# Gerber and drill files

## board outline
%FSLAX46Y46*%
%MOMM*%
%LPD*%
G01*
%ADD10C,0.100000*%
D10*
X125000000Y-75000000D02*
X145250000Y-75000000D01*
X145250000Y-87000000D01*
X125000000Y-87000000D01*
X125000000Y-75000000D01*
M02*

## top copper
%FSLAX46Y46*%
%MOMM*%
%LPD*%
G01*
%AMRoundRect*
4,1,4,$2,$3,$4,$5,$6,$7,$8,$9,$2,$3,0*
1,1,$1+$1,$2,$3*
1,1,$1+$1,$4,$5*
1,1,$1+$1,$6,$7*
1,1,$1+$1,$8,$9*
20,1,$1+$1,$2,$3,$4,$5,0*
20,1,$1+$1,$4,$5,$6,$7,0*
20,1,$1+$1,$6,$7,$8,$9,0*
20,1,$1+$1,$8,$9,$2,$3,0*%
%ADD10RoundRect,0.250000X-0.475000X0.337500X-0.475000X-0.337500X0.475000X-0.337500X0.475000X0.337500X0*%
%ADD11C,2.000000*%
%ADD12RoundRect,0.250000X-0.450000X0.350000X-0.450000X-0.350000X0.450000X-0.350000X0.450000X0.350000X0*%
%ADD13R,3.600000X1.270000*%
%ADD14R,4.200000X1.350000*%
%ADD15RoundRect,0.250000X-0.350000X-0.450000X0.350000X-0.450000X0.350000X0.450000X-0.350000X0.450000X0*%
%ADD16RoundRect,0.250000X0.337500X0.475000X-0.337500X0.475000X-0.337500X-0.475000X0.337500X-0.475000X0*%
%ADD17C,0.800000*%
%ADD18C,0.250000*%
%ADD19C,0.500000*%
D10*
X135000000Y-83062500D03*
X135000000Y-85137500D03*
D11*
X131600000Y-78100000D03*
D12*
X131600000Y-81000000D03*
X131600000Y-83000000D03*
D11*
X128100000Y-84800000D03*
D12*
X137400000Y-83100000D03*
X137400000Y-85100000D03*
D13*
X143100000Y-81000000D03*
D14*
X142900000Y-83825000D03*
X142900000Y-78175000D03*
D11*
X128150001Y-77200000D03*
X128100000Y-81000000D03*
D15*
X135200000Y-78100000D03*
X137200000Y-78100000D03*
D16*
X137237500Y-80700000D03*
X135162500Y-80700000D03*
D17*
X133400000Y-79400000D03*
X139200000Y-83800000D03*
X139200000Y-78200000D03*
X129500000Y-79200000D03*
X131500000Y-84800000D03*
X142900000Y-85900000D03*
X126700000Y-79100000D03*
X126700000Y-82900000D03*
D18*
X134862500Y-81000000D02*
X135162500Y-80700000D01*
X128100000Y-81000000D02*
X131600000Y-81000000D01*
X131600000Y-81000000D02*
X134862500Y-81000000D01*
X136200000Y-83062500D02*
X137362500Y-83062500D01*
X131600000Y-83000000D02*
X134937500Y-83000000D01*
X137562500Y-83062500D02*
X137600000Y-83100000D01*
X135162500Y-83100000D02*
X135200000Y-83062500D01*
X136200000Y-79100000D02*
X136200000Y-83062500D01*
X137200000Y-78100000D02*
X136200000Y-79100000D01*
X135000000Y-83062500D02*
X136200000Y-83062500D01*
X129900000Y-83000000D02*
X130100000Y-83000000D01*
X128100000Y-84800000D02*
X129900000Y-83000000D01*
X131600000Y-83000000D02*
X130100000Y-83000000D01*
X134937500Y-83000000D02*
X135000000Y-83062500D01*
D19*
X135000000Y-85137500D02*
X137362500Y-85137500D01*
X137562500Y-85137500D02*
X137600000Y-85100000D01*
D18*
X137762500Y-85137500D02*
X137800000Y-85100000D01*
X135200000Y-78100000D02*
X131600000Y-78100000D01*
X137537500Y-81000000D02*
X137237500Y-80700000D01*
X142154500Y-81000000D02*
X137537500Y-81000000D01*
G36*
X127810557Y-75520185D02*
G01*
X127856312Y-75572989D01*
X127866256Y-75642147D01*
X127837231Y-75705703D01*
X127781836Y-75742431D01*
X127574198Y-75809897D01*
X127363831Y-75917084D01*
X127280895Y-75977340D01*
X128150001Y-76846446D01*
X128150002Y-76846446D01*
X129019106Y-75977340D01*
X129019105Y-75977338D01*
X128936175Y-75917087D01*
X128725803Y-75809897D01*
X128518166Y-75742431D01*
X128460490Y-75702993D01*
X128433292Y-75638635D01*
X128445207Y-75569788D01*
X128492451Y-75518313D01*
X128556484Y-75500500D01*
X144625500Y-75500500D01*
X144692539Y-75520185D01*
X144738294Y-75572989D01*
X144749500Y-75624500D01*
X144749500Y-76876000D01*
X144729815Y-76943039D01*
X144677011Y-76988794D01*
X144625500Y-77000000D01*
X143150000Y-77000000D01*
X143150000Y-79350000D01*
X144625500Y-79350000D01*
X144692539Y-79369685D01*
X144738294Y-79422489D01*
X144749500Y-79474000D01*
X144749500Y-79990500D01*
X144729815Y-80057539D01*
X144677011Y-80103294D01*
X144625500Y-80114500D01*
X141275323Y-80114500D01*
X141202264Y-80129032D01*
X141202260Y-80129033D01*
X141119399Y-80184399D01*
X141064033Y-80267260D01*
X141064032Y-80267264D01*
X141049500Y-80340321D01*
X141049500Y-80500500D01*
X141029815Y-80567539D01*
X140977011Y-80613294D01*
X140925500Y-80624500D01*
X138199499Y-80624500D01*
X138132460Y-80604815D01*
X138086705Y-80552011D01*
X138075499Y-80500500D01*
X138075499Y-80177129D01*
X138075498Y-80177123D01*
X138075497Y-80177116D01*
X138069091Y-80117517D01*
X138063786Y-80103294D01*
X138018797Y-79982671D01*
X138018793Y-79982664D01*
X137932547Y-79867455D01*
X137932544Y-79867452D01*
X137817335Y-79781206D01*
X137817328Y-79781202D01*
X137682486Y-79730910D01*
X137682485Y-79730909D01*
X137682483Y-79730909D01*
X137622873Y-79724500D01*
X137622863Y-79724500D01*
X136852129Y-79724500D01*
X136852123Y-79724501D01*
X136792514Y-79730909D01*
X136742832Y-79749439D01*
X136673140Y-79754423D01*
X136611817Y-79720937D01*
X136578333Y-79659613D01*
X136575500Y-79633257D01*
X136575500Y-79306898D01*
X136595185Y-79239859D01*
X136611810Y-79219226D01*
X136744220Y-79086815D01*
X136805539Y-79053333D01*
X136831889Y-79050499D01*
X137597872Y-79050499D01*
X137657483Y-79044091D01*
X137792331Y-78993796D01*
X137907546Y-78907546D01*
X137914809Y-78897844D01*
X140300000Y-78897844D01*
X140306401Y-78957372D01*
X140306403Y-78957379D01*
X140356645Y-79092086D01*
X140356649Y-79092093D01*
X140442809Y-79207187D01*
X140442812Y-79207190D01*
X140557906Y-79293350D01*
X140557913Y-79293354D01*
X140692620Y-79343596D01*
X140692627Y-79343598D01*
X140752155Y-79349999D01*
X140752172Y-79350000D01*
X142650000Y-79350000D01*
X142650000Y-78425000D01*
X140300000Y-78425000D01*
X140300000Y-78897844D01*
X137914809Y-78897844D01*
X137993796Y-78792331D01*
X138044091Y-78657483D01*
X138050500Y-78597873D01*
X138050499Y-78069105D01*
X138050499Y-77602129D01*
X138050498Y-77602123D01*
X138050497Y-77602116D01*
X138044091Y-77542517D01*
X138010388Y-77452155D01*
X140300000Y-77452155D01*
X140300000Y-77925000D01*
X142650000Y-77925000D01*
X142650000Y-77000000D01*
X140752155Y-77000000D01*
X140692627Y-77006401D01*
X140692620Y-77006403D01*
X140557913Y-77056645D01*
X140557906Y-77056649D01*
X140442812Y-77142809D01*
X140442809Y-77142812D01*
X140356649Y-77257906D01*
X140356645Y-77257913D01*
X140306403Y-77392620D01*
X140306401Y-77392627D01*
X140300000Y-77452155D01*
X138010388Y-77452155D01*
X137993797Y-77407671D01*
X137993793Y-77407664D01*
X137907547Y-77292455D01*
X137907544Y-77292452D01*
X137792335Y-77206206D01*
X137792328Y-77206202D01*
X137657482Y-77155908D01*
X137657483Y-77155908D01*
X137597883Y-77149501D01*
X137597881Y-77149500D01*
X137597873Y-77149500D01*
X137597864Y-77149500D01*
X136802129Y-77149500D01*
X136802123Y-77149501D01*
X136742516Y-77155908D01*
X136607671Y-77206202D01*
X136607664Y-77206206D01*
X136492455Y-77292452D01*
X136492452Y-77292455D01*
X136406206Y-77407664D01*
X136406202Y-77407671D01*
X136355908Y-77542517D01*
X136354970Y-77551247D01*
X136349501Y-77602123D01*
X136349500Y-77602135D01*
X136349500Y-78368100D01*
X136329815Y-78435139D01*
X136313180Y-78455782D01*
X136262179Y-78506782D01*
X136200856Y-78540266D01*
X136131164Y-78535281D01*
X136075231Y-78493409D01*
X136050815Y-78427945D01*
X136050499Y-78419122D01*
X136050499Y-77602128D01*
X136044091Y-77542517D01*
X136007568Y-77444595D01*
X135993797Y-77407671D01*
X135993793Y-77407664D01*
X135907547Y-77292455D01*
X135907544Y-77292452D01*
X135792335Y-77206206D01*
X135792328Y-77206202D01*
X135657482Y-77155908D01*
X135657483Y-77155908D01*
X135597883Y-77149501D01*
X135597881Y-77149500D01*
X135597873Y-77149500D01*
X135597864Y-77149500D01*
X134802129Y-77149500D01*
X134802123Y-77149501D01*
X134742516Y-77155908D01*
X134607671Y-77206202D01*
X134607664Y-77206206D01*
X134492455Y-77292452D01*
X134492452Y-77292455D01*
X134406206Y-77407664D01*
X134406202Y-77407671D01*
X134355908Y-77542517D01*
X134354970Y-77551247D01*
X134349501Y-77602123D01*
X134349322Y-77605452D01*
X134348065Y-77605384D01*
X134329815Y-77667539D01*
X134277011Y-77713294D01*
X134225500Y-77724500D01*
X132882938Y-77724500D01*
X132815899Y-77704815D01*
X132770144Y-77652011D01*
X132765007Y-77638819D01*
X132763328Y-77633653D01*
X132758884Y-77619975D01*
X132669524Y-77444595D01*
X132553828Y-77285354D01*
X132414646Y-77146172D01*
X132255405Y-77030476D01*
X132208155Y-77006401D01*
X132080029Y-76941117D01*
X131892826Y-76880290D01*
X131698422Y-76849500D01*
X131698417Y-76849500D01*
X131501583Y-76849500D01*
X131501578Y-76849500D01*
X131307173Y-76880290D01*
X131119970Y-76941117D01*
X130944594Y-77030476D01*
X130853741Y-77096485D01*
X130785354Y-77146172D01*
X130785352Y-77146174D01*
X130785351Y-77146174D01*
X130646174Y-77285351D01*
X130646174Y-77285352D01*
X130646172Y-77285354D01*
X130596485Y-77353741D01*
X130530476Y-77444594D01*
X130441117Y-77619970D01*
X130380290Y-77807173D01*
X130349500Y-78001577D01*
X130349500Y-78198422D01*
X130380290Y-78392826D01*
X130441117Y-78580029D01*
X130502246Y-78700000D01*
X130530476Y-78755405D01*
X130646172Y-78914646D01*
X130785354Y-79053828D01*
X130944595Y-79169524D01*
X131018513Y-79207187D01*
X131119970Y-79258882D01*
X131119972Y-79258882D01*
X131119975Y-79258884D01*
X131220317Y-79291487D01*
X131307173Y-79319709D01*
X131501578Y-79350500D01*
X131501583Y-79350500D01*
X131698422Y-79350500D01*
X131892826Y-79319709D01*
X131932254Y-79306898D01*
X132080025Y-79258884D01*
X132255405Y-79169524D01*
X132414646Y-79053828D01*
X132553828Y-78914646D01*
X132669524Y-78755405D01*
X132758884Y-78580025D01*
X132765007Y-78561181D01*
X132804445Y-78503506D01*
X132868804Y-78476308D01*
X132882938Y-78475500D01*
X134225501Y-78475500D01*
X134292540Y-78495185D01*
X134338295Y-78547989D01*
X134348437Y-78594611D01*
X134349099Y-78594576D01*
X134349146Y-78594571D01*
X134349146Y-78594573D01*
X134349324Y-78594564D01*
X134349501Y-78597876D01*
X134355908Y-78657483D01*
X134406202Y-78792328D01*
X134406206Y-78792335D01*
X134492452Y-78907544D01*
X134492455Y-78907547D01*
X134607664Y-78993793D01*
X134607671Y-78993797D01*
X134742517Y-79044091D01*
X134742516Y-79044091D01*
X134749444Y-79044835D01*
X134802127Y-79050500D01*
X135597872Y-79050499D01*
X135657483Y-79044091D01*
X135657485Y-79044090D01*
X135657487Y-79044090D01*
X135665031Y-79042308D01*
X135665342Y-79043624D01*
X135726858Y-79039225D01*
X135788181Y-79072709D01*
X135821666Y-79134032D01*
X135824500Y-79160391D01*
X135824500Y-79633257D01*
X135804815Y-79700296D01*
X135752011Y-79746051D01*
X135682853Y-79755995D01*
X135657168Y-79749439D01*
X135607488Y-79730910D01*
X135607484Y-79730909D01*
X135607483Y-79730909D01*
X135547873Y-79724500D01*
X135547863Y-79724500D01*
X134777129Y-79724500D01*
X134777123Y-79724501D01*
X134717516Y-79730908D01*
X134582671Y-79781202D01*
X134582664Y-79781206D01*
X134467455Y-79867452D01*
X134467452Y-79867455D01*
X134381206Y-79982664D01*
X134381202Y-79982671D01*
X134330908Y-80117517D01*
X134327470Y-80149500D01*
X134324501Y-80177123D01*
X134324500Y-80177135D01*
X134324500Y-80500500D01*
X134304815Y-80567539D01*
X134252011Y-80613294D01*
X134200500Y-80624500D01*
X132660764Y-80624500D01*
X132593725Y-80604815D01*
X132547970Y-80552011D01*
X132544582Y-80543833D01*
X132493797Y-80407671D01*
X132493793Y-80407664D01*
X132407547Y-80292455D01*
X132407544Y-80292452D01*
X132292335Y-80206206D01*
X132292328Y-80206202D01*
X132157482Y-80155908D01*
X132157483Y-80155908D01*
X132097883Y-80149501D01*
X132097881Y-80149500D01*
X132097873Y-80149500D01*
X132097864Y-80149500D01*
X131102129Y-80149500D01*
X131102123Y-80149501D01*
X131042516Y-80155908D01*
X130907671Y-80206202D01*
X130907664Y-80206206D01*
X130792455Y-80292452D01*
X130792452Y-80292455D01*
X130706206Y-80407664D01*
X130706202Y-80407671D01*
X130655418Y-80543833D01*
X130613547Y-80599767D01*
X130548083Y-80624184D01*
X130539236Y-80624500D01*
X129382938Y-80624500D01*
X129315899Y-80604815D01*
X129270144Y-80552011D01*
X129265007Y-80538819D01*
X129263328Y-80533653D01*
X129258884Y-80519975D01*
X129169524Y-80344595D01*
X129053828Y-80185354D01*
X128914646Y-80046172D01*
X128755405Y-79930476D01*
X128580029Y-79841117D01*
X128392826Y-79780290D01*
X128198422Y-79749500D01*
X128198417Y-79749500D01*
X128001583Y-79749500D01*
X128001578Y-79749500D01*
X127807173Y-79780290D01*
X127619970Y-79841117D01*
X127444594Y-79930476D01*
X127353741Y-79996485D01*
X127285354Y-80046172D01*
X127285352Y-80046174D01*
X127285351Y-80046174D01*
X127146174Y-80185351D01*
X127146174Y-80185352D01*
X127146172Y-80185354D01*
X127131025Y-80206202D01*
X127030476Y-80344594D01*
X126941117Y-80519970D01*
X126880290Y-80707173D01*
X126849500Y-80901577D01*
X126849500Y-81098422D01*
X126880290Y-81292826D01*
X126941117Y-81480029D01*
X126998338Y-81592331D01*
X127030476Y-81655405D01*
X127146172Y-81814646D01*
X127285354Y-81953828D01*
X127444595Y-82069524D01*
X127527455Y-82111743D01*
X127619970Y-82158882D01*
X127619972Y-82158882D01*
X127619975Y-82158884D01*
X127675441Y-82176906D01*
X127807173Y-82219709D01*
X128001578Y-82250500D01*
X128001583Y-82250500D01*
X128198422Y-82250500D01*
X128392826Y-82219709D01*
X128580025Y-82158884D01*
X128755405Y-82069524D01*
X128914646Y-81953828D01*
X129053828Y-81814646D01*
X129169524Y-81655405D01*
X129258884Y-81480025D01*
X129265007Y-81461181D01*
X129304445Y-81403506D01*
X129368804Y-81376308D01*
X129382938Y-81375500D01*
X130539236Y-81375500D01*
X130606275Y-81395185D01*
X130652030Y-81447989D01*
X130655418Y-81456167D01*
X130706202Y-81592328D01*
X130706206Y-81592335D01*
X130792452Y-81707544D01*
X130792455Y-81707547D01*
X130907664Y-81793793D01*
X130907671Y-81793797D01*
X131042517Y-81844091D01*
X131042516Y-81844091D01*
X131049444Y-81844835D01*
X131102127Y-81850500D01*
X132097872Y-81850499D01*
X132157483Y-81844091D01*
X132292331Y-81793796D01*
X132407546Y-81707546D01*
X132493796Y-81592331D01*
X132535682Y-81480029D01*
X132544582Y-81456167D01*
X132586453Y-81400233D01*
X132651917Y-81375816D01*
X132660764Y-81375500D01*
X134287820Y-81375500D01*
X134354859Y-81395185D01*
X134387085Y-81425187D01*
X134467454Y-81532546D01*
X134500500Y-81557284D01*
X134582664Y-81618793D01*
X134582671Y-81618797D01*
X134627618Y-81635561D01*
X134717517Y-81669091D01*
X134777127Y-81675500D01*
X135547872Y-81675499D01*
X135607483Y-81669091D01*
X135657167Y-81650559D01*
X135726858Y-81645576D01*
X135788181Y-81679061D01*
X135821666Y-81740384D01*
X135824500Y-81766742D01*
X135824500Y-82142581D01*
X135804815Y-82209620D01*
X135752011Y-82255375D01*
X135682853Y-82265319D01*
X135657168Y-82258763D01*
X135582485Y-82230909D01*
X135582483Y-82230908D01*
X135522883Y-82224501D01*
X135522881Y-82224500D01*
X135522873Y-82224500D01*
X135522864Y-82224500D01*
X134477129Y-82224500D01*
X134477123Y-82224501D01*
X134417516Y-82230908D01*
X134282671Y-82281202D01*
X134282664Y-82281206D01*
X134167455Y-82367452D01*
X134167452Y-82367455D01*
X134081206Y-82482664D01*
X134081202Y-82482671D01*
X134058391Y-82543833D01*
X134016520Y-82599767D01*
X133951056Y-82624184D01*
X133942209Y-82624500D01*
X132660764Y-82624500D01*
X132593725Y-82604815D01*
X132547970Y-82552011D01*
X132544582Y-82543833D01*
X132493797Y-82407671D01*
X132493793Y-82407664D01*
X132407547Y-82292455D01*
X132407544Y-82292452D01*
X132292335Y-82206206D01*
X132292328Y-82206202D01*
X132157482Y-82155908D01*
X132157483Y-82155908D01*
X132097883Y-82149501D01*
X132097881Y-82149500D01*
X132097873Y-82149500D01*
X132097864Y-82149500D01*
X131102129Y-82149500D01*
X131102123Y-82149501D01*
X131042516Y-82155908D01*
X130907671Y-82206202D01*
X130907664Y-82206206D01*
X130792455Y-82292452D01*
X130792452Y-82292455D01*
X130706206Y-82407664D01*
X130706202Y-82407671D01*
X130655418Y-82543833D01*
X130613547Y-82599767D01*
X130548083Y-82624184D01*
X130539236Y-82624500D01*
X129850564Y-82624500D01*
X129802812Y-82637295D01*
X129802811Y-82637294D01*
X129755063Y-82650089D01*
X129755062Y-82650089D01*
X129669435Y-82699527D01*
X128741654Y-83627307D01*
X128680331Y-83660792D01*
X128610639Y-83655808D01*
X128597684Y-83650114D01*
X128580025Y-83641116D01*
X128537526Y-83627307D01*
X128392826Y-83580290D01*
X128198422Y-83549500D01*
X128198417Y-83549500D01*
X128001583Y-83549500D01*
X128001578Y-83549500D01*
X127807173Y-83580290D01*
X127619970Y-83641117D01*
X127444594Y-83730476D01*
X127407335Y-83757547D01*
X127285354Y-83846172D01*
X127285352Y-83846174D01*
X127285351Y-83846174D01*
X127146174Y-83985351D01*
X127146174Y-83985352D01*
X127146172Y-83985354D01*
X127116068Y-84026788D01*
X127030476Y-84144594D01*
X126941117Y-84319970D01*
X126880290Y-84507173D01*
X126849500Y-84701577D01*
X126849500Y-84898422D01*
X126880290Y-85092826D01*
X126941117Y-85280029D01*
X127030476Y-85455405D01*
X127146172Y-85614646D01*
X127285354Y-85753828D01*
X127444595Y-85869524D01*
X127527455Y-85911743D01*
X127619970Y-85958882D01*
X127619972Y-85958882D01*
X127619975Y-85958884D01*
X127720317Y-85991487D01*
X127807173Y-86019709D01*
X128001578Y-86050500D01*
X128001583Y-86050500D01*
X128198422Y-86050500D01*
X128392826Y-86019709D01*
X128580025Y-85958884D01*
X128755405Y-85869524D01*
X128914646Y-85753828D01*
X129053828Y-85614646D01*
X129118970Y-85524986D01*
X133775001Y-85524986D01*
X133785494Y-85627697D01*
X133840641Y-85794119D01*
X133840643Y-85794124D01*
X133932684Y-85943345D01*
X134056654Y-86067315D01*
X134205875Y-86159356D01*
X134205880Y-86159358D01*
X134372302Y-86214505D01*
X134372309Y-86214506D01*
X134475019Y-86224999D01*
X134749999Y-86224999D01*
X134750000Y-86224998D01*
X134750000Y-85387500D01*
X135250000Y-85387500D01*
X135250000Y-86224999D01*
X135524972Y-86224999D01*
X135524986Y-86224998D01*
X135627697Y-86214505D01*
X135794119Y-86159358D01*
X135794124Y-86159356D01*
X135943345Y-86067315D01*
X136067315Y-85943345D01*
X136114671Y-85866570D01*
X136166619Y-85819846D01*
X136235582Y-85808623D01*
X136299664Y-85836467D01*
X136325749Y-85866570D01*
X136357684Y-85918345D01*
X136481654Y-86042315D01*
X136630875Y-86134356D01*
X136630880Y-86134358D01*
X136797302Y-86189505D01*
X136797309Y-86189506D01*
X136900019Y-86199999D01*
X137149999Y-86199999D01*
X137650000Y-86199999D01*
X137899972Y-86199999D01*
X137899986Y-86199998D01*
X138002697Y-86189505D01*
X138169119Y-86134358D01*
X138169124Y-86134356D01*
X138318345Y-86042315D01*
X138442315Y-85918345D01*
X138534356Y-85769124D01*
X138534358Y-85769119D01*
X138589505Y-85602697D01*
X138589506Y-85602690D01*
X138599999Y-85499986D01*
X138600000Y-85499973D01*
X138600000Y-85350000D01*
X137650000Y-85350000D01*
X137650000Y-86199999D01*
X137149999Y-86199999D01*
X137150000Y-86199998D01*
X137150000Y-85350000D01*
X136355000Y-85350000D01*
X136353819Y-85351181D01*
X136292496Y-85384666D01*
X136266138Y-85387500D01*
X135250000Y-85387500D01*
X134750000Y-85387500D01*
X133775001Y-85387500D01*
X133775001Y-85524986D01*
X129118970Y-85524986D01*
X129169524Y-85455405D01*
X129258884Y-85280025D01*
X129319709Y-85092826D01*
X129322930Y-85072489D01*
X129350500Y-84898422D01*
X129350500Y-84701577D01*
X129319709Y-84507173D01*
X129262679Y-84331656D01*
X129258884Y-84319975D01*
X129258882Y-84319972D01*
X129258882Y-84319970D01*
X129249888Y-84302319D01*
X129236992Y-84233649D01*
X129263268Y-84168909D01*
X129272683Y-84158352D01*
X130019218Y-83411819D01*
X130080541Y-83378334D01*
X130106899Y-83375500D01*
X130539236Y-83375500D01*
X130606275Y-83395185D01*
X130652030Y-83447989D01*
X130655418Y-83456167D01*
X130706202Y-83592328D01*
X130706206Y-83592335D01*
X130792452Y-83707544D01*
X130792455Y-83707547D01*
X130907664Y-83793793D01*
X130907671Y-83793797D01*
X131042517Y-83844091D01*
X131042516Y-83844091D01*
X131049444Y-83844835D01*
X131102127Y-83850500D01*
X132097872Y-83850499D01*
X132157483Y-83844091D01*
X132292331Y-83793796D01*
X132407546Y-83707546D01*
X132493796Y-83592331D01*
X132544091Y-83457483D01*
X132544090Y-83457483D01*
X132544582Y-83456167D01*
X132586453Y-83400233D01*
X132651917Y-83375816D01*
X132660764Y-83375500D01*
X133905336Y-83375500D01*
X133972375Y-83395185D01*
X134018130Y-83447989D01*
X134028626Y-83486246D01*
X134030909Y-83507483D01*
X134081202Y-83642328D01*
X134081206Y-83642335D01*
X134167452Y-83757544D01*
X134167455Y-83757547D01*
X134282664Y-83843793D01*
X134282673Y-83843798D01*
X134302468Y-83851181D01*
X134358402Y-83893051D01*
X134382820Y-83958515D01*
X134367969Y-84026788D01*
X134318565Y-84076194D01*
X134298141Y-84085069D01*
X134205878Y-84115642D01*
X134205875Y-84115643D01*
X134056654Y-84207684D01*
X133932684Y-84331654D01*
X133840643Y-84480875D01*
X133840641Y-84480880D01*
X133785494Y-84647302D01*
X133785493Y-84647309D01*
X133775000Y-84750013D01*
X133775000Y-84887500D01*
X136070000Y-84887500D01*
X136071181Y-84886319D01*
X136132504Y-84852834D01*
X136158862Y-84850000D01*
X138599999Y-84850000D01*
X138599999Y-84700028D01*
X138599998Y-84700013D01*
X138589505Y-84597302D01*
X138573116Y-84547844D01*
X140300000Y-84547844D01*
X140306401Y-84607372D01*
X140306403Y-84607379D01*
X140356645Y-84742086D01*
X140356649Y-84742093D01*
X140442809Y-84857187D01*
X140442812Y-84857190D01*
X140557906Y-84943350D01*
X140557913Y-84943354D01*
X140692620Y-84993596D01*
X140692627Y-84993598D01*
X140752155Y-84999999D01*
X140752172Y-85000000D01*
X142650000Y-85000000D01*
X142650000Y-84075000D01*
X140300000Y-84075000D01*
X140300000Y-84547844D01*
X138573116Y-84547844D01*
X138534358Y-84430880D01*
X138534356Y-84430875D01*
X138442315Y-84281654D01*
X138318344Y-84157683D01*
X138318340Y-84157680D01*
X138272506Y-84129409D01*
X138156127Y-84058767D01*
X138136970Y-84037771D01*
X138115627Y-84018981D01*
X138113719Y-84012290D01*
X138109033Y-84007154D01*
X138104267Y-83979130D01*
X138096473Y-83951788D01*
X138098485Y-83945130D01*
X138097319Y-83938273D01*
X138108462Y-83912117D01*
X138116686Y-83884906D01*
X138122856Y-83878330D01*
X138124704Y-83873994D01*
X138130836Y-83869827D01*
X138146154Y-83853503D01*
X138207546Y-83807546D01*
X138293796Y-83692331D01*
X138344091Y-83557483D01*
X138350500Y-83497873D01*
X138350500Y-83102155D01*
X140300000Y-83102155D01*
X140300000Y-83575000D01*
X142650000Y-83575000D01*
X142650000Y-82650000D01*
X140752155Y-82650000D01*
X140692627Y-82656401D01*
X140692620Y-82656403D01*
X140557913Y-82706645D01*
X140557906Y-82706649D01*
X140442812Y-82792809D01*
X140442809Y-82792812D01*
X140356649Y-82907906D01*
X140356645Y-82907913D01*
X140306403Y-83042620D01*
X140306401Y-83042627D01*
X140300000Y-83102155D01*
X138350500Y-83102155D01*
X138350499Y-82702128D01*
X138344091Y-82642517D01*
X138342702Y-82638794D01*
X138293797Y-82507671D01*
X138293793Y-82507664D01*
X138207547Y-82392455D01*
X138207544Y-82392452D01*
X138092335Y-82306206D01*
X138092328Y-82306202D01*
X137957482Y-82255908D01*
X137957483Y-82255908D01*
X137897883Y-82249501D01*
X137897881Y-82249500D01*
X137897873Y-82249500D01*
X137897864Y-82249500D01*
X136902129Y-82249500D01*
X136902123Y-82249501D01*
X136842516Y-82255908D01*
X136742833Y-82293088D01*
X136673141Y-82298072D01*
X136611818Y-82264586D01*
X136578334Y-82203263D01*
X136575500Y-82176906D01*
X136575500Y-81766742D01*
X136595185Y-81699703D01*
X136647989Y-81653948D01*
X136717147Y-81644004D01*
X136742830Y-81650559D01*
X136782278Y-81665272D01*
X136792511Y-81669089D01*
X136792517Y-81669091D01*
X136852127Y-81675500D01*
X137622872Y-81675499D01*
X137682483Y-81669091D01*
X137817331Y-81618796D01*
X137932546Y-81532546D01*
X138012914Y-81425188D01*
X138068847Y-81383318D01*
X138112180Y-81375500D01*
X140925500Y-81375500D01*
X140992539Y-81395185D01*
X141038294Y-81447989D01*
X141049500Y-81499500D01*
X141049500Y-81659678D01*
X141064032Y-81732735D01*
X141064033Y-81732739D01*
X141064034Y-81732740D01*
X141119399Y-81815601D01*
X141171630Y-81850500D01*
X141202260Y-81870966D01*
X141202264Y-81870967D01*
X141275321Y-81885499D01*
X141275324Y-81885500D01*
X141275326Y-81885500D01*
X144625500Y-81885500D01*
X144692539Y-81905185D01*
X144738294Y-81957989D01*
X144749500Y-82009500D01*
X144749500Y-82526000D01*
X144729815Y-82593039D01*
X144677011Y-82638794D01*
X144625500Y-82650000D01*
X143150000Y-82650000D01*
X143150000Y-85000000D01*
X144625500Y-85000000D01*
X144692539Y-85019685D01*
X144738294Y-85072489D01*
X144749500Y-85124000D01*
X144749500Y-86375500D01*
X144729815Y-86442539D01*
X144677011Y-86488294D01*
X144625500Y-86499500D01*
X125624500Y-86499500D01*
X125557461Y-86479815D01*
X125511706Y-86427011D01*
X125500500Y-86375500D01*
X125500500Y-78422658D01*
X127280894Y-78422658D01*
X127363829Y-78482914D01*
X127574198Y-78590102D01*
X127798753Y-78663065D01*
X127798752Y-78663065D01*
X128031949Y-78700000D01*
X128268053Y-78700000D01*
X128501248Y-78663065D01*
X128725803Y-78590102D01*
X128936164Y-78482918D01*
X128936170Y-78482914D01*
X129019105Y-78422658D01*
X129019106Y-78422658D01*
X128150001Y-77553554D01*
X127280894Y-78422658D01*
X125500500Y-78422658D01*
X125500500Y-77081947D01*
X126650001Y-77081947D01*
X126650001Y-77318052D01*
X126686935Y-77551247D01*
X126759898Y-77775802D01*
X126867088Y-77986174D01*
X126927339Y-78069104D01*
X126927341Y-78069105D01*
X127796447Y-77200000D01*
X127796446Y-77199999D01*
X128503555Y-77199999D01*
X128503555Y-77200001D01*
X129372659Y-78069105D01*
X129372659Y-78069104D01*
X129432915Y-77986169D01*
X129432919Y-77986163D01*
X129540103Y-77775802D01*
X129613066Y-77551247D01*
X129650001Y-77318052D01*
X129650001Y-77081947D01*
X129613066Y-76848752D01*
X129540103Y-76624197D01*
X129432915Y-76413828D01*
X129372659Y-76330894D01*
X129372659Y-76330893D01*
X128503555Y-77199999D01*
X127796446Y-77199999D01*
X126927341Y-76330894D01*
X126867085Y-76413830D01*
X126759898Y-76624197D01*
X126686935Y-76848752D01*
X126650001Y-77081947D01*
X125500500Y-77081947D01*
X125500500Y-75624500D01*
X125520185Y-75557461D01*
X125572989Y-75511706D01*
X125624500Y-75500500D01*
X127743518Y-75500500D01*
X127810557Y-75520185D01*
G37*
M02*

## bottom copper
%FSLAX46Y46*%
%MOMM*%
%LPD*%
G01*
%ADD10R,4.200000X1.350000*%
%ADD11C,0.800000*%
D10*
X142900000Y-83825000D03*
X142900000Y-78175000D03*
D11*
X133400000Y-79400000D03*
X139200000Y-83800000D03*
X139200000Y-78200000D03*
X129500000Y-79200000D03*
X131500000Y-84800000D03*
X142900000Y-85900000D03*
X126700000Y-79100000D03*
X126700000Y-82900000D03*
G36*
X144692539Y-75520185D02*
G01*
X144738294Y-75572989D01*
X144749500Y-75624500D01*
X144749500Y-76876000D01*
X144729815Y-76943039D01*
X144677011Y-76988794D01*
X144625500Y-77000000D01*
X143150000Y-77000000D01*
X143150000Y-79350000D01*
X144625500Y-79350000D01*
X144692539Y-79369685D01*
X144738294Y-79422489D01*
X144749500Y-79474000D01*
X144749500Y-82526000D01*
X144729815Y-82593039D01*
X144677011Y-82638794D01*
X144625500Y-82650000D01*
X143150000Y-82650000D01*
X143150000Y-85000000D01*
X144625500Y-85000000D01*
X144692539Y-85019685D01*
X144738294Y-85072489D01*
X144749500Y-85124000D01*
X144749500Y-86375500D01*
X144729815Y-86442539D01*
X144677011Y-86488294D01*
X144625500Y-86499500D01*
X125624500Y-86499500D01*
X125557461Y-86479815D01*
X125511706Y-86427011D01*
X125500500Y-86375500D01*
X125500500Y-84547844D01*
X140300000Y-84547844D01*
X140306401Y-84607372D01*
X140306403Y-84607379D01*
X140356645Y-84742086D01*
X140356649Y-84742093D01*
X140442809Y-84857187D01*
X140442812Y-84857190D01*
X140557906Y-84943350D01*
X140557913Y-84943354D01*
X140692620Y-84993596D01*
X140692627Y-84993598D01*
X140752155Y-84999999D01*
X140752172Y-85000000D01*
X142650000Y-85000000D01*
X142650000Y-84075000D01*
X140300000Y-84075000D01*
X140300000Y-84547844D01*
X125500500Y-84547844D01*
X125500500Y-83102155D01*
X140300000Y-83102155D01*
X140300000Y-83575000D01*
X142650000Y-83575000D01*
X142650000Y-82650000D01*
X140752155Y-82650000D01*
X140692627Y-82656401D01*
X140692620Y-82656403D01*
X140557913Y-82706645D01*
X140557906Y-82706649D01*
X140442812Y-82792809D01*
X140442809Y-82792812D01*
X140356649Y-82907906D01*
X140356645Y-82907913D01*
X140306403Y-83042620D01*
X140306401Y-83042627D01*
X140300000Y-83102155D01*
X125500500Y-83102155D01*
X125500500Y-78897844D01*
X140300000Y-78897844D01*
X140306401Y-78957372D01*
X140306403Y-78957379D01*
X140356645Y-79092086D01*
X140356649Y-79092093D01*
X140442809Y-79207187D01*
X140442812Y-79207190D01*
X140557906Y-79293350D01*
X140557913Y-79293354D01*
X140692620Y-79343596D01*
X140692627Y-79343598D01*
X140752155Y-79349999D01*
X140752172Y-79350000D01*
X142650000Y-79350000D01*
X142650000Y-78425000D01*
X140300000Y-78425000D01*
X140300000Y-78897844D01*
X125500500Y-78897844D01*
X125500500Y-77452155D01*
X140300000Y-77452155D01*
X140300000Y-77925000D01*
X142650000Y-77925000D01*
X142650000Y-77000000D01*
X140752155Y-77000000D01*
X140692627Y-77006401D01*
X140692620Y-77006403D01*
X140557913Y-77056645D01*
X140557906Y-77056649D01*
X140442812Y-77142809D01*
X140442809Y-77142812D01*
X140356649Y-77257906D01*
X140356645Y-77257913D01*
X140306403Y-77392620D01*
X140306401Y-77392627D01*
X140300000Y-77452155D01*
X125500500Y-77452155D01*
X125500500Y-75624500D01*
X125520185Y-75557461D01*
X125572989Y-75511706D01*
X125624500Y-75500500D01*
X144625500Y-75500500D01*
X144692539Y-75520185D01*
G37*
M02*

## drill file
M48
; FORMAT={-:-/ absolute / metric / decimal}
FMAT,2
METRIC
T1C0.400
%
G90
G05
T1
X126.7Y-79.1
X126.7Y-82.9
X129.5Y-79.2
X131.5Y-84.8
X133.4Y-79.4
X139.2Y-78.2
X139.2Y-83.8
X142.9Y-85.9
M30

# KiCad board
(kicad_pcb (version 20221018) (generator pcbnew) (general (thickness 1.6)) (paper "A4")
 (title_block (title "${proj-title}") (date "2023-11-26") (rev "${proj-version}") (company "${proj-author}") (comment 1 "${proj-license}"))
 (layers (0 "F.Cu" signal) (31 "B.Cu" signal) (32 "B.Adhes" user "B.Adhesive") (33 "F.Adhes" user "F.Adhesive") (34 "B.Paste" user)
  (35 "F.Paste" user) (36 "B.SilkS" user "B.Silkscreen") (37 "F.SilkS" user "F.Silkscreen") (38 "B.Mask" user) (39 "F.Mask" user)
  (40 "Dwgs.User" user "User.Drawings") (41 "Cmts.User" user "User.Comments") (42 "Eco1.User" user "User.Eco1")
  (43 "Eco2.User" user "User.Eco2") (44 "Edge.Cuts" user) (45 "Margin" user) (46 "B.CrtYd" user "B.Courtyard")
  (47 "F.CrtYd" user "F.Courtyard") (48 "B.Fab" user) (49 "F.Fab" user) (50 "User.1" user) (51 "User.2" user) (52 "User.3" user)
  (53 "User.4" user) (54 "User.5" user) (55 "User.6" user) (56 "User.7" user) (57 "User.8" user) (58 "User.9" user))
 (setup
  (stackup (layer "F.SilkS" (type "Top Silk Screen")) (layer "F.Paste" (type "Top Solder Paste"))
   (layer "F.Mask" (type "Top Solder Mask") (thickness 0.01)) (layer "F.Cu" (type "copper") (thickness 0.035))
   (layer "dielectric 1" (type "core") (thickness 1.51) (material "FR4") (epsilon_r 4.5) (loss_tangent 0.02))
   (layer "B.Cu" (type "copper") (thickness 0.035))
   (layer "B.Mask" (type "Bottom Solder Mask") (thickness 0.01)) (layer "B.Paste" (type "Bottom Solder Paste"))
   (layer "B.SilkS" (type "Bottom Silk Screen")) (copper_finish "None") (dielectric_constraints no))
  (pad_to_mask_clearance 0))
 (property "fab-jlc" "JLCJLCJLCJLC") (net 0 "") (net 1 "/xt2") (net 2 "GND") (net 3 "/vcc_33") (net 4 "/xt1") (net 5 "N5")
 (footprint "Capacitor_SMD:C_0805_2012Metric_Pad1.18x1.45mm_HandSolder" (layer "F.Cu") (at 135 84.1 -90)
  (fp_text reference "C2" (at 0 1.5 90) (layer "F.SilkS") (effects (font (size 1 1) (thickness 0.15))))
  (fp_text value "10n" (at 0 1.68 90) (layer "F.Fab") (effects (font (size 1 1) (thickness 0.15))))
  (pad "1" smd roundrect (at -1.0375 0 270) (size 1.175 1.45) (layers "F.Cu" "F.Paste" "F.Mask") (roundrect_rratio 0.2127659574)
   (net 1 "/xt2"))
  (pad "2" smd roundrect (at 1.0375 0 270) (size 1.175 1.45) (layers "F.Cu" "F.Paste" "F.Mask") (roundrect_rratio 0.2127659574)
   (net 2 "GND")))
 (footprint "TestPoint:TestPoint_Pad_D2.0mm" (layer "F.Cu") (at 131.6 78.1)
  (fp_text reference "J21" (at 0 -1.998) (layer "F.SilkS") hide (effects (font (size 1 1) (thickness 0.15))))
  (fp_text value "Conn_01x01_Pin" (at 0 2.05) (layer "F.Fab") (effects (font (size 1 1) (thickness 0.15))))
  (pad "1" smd circle (at 0 0) (size 2 2) (layers "F.Cu" "F.Mask") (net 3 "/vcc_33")))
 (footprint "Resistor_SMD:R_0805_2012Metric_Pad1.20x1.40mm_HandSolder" (layer "F.Cu") (at 131.6 82 -90)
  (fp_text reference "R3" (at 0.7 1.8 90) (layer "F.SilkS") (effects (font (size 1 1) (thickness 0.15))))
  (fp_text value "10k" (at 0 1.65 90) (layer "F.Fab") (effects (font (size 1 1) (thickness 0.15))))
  (pad "1" smd roundrect (at -1 0 270) (size 1.2 1.4) (layers "F.Cu" "F.Paste" "F.Mask") (roundrect_rratio 0.2083333333) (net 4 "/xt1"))
  (pad "2" smd roundrect (at 1 0 270) (size 1.2 1.4) (layers "F.Cu" "F.Paste" "F.Mask") (roundrect_rratio 0.2083333333) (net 1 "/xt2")))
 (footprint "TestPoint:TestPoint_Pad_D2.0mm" (layer "F.Cu") (at 128.1 84.8)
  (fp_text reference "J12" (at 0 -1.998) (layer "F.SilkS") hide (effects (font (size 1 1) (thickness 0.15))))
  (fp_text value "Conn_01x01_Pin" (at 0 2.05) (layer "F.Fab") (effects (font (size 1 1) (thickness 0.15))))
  (pad "1" smd circle (at 0 0) (size 2 2) (layers "F.Cu" "F.Mask") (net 1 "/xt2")))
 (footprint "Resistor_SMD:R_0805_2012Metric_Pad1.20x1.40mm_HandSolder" (layer "F.Cu") (at 137.4 84.1 -90)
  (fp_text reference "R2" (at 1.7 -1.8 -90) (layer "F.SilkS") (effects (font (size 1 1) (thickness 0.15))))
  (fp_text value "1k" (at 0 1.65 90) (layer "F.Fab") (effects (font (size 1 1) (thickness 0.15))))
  (pad "1" smd roundrect (at -1 0 270) (size 1.2 1.4) (layers "F.Cu" "F.Paste" "F.Mask") (roundrect_rratio 0.2083333333) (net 1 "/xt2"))
  (pad "2" smd roundrect (at 1 0 270) (size 1.2 1.4) (layers "F.Cu" "F.Paste" "F.Mask") (roundrect_rratio 0.2083333333) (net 2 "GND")))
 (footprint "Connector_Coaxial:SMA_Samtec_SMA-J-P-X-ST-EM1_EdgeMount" (layer "F.Cu") (at 142.9 81 90)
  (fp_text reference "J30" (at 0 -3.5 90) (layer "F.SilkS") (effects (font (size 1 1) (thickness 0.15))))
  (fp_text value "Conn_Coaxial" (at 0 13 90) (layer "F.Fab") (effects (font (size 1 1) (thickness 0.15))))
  (pad "1" smd rect (at 0 0.2 90) (size 1.27 3.6) (layers "F.Cu" "F.Paste" "F.Mask") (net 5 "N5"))
  (pad "2" smd rect (at -2.825 0 90) (size 1.35 4.2) (layers "F.Cu" "F.Paste" "F.Mask") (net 2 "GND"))
  (pad "2" smd rect (at -2.825 0 90) (size 1.35 4.2) (layers "B.Cu" "B.Paste" "B.Mask") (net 2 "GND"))
  (pad "2" smd rect (at 2.825 0 90) (size 1.35 4.2) (layers "F.Cu" "F.Paste" "F.Mask") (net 2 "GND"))
  (pad "2" smd rect (at 2.825 0 90) (size 1.35 4.2) (layers "B.Cu" "B.Paste" "B.Mask") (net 2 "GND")))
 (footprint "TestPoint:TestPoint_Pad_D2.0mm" (layer "F.Cu") (at 128.150001 77.2)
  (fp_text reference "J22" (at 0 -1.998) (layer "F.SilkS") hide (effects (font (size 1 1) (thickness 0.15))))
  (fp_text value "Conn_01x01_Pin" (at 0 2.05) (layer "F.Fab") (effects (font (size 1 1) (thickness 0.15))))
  (pad "1" smd circle (at 0 0) (size 2 2) (layers "F.Cu" "F.Mask") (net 2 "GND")))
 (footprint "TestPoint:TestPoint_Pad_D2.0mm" (layer "F.Cu") (at 128.1 81)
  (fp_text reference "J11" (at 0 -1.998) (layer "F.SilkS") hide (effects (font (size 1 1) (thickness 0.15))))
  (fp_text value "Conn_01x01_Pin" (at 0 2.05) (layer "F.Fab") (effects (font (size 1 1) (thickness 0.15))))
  (pad "1" smd circle (at 0 0) (size 2 2) (layers "F.Cu" "F.Mask") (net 4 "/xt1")))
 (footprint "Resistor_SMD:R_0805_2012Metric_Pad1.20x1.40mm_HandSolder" (layer "F.Cu") (at 136.2 78.1)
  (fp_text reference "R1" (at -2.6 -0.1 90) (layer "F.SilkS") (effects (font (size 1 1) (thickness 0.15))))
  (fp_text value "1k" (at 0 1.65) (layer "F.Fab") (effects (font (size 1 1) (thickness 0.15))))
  (pad "1" smd roundrect (at -1 0) (size 1.2 1.4) (layers "F.Cu" "F.Paste" "F.Mask") (roundrect_rratio 0.2083333333) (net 3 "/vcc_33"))
  (pad "2" smd roundrect (at 1 0) (size 1.2 1.4) (layers "F.Cu" "F.Paste" "F.Mask") (roundrect_rratio 0.2083333333) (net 1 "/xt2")))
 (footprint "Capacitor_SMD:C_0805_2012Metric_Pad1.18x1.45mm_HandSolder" (layer "F.Cu") (at 136.2 80.7 180)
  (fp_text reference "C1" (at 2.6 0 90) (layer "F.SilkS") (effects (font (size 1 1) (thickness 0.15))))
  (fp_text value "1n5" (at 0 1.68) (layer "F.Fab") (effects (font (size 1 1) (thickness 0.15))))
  (pad "1" smd roundrect (at -1.0375 0 180) (size 1.175 1.45) (layers "F.Cu" "F.Paste" "F.Mask") (roundrect_rratio 0.2127659574)
   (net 5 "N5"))
  (pad "2" smd roundrect (at 1.0375 0 180) (size 1.175 1.45) (layers "F.Cu" "F.Paste" "F.Mask") (roundrect_rratio 0.2127659574)
   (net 4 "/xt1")))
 (gr_rect (start 125 75) (end 145.25 87) (stroke (width 0.1) (type default)) (fill none) (layer "Edge.Cuts"))
 (segment (start 134.8625 81) (end 135.1625 80.7) (width 0.25) (layer "F.Cu") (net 4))
 (segment (start 128.1 81) (end 131.6 81) (width 0.25) (layer "F.Cu") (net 4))
 (segment (start 131.6 81) (end 134.8625 81) (width 0.25) (layer "F.Cu") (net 4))
 (segment (start 136.2 83.0625) (end 137.3625 83.0625) (width 0.25) (layer "F.Cu") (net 1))
 (segment (start 131.6 83) (end 134.9375 83) (width 0.25) (layer "F.Cu") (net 1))
 (segment (start 137.5625 83.0625) (end 137.6 83.1) (width 0.25) (layer "F.Cu") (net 1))
 (segment (start 135.1625 83.1) (end 135.2 83.0625) (width 0.25) (layer "F.Cu") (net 1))
 (segment (start 136.2 79.1) (end 136.2 83.0625) (width 0.25) (layer "F.Cu") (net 1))
 (segment (start 137.2 78.1) (end 136.2 79.1) (width 0.25) (layer "F.Cu") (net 1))
 (segment (start 135 83.0625) (end 136.2 83.0625) (width 0.25) (layer "F.Cu") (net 1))
 (segment (start 129.9 83) (end 130.1 83) (width 0.25) (layer "F.Cu") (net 1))
 (segment (start 128.1 84.8) (end 129.9 83) (width 0.25) (layer "F.Cu") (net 1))
 (segment (start 131.6 83) (end 130.1 83) (width 0.25) (layer "F.Cu") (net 1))
 (segment (start 134.9375 83) (end 135 83.0625) (width 0.25) (layer "F.Cu") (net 1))
 (segment (start 135 85.1375) (end 137.3625 85.1375) (width 0.5) (layer "F.Cu") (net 2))
 (segment (start 137.5625 85.1375) (end 137.6 85.1) (width 0.5) (layer "F.Cu") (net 2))
 (segment (start 137.7625 85.1375) (end 137.8 85.1) (width 0.25) (layer "F.Cu") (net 2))
 (via (at 133.4 79.4) (size 0.8) (drill 0.4) (layers "F.Cu" "B.Cu") (free) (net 2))
 (via (at 139.2 83.8) (size 0.8) (drill 0.4) (layers "F.Cu" "B.Cu") (free) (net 2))
 (via (at 139.2 78.2) (size 0.8) (drill 0.4) (layers "F.Cu" "B.Cu") (free) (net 2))
 (via (at 129.5 79.2) (size 0.8) (drill 0.4) (layers "F.Cu" "B.Cu") (free) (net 2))
 (via (at 131.5 84.8) (size 0.8) (drill 0.4) (layers "F.Cu" "B.Cu") (free) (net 2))
 (via (at 142.9 85.9) (size 0.8) (drill 0.4) (layers "F.Cu" "B.Cu") (free) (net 2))
 (via (at 126.7 79.1) (size 0.8) (drill 0.4) (layers "F.Cu" "B.Cu") (free) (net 2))
 (via (at 126.7 82.9) (size 0.8) (drill 0.4) (layers "F.Cu" "B.Cu") (free) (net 2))
 (segment (start 135.2 78.1) (end 131.6 78.1) (width 0.25) (layer "F.Cu") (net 3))
 (segment (start 137.5375 81) (end 137.2375 80.7) (width 0.25) (layer "F.Cu") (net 5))
 (segment (start 142.1545 81) (end 137.5375 81) (width 0.25) (layer "F.Cu") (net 5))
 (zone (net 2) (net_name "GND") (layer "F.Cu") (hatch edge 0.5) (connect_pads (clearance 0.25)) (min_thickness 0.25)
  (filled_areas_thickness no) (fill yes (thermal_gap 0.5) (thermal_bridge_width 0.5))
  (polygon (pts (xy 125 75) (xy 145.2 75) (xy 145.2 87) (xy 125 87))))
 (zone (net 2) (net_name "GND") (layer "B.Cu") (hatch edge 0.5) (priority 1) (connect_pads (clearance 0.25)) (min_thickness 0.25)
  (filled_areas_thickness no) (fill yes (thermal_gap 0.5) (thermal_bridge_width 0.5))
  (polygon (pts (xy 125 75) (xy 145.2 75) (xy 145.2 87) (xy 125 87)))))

